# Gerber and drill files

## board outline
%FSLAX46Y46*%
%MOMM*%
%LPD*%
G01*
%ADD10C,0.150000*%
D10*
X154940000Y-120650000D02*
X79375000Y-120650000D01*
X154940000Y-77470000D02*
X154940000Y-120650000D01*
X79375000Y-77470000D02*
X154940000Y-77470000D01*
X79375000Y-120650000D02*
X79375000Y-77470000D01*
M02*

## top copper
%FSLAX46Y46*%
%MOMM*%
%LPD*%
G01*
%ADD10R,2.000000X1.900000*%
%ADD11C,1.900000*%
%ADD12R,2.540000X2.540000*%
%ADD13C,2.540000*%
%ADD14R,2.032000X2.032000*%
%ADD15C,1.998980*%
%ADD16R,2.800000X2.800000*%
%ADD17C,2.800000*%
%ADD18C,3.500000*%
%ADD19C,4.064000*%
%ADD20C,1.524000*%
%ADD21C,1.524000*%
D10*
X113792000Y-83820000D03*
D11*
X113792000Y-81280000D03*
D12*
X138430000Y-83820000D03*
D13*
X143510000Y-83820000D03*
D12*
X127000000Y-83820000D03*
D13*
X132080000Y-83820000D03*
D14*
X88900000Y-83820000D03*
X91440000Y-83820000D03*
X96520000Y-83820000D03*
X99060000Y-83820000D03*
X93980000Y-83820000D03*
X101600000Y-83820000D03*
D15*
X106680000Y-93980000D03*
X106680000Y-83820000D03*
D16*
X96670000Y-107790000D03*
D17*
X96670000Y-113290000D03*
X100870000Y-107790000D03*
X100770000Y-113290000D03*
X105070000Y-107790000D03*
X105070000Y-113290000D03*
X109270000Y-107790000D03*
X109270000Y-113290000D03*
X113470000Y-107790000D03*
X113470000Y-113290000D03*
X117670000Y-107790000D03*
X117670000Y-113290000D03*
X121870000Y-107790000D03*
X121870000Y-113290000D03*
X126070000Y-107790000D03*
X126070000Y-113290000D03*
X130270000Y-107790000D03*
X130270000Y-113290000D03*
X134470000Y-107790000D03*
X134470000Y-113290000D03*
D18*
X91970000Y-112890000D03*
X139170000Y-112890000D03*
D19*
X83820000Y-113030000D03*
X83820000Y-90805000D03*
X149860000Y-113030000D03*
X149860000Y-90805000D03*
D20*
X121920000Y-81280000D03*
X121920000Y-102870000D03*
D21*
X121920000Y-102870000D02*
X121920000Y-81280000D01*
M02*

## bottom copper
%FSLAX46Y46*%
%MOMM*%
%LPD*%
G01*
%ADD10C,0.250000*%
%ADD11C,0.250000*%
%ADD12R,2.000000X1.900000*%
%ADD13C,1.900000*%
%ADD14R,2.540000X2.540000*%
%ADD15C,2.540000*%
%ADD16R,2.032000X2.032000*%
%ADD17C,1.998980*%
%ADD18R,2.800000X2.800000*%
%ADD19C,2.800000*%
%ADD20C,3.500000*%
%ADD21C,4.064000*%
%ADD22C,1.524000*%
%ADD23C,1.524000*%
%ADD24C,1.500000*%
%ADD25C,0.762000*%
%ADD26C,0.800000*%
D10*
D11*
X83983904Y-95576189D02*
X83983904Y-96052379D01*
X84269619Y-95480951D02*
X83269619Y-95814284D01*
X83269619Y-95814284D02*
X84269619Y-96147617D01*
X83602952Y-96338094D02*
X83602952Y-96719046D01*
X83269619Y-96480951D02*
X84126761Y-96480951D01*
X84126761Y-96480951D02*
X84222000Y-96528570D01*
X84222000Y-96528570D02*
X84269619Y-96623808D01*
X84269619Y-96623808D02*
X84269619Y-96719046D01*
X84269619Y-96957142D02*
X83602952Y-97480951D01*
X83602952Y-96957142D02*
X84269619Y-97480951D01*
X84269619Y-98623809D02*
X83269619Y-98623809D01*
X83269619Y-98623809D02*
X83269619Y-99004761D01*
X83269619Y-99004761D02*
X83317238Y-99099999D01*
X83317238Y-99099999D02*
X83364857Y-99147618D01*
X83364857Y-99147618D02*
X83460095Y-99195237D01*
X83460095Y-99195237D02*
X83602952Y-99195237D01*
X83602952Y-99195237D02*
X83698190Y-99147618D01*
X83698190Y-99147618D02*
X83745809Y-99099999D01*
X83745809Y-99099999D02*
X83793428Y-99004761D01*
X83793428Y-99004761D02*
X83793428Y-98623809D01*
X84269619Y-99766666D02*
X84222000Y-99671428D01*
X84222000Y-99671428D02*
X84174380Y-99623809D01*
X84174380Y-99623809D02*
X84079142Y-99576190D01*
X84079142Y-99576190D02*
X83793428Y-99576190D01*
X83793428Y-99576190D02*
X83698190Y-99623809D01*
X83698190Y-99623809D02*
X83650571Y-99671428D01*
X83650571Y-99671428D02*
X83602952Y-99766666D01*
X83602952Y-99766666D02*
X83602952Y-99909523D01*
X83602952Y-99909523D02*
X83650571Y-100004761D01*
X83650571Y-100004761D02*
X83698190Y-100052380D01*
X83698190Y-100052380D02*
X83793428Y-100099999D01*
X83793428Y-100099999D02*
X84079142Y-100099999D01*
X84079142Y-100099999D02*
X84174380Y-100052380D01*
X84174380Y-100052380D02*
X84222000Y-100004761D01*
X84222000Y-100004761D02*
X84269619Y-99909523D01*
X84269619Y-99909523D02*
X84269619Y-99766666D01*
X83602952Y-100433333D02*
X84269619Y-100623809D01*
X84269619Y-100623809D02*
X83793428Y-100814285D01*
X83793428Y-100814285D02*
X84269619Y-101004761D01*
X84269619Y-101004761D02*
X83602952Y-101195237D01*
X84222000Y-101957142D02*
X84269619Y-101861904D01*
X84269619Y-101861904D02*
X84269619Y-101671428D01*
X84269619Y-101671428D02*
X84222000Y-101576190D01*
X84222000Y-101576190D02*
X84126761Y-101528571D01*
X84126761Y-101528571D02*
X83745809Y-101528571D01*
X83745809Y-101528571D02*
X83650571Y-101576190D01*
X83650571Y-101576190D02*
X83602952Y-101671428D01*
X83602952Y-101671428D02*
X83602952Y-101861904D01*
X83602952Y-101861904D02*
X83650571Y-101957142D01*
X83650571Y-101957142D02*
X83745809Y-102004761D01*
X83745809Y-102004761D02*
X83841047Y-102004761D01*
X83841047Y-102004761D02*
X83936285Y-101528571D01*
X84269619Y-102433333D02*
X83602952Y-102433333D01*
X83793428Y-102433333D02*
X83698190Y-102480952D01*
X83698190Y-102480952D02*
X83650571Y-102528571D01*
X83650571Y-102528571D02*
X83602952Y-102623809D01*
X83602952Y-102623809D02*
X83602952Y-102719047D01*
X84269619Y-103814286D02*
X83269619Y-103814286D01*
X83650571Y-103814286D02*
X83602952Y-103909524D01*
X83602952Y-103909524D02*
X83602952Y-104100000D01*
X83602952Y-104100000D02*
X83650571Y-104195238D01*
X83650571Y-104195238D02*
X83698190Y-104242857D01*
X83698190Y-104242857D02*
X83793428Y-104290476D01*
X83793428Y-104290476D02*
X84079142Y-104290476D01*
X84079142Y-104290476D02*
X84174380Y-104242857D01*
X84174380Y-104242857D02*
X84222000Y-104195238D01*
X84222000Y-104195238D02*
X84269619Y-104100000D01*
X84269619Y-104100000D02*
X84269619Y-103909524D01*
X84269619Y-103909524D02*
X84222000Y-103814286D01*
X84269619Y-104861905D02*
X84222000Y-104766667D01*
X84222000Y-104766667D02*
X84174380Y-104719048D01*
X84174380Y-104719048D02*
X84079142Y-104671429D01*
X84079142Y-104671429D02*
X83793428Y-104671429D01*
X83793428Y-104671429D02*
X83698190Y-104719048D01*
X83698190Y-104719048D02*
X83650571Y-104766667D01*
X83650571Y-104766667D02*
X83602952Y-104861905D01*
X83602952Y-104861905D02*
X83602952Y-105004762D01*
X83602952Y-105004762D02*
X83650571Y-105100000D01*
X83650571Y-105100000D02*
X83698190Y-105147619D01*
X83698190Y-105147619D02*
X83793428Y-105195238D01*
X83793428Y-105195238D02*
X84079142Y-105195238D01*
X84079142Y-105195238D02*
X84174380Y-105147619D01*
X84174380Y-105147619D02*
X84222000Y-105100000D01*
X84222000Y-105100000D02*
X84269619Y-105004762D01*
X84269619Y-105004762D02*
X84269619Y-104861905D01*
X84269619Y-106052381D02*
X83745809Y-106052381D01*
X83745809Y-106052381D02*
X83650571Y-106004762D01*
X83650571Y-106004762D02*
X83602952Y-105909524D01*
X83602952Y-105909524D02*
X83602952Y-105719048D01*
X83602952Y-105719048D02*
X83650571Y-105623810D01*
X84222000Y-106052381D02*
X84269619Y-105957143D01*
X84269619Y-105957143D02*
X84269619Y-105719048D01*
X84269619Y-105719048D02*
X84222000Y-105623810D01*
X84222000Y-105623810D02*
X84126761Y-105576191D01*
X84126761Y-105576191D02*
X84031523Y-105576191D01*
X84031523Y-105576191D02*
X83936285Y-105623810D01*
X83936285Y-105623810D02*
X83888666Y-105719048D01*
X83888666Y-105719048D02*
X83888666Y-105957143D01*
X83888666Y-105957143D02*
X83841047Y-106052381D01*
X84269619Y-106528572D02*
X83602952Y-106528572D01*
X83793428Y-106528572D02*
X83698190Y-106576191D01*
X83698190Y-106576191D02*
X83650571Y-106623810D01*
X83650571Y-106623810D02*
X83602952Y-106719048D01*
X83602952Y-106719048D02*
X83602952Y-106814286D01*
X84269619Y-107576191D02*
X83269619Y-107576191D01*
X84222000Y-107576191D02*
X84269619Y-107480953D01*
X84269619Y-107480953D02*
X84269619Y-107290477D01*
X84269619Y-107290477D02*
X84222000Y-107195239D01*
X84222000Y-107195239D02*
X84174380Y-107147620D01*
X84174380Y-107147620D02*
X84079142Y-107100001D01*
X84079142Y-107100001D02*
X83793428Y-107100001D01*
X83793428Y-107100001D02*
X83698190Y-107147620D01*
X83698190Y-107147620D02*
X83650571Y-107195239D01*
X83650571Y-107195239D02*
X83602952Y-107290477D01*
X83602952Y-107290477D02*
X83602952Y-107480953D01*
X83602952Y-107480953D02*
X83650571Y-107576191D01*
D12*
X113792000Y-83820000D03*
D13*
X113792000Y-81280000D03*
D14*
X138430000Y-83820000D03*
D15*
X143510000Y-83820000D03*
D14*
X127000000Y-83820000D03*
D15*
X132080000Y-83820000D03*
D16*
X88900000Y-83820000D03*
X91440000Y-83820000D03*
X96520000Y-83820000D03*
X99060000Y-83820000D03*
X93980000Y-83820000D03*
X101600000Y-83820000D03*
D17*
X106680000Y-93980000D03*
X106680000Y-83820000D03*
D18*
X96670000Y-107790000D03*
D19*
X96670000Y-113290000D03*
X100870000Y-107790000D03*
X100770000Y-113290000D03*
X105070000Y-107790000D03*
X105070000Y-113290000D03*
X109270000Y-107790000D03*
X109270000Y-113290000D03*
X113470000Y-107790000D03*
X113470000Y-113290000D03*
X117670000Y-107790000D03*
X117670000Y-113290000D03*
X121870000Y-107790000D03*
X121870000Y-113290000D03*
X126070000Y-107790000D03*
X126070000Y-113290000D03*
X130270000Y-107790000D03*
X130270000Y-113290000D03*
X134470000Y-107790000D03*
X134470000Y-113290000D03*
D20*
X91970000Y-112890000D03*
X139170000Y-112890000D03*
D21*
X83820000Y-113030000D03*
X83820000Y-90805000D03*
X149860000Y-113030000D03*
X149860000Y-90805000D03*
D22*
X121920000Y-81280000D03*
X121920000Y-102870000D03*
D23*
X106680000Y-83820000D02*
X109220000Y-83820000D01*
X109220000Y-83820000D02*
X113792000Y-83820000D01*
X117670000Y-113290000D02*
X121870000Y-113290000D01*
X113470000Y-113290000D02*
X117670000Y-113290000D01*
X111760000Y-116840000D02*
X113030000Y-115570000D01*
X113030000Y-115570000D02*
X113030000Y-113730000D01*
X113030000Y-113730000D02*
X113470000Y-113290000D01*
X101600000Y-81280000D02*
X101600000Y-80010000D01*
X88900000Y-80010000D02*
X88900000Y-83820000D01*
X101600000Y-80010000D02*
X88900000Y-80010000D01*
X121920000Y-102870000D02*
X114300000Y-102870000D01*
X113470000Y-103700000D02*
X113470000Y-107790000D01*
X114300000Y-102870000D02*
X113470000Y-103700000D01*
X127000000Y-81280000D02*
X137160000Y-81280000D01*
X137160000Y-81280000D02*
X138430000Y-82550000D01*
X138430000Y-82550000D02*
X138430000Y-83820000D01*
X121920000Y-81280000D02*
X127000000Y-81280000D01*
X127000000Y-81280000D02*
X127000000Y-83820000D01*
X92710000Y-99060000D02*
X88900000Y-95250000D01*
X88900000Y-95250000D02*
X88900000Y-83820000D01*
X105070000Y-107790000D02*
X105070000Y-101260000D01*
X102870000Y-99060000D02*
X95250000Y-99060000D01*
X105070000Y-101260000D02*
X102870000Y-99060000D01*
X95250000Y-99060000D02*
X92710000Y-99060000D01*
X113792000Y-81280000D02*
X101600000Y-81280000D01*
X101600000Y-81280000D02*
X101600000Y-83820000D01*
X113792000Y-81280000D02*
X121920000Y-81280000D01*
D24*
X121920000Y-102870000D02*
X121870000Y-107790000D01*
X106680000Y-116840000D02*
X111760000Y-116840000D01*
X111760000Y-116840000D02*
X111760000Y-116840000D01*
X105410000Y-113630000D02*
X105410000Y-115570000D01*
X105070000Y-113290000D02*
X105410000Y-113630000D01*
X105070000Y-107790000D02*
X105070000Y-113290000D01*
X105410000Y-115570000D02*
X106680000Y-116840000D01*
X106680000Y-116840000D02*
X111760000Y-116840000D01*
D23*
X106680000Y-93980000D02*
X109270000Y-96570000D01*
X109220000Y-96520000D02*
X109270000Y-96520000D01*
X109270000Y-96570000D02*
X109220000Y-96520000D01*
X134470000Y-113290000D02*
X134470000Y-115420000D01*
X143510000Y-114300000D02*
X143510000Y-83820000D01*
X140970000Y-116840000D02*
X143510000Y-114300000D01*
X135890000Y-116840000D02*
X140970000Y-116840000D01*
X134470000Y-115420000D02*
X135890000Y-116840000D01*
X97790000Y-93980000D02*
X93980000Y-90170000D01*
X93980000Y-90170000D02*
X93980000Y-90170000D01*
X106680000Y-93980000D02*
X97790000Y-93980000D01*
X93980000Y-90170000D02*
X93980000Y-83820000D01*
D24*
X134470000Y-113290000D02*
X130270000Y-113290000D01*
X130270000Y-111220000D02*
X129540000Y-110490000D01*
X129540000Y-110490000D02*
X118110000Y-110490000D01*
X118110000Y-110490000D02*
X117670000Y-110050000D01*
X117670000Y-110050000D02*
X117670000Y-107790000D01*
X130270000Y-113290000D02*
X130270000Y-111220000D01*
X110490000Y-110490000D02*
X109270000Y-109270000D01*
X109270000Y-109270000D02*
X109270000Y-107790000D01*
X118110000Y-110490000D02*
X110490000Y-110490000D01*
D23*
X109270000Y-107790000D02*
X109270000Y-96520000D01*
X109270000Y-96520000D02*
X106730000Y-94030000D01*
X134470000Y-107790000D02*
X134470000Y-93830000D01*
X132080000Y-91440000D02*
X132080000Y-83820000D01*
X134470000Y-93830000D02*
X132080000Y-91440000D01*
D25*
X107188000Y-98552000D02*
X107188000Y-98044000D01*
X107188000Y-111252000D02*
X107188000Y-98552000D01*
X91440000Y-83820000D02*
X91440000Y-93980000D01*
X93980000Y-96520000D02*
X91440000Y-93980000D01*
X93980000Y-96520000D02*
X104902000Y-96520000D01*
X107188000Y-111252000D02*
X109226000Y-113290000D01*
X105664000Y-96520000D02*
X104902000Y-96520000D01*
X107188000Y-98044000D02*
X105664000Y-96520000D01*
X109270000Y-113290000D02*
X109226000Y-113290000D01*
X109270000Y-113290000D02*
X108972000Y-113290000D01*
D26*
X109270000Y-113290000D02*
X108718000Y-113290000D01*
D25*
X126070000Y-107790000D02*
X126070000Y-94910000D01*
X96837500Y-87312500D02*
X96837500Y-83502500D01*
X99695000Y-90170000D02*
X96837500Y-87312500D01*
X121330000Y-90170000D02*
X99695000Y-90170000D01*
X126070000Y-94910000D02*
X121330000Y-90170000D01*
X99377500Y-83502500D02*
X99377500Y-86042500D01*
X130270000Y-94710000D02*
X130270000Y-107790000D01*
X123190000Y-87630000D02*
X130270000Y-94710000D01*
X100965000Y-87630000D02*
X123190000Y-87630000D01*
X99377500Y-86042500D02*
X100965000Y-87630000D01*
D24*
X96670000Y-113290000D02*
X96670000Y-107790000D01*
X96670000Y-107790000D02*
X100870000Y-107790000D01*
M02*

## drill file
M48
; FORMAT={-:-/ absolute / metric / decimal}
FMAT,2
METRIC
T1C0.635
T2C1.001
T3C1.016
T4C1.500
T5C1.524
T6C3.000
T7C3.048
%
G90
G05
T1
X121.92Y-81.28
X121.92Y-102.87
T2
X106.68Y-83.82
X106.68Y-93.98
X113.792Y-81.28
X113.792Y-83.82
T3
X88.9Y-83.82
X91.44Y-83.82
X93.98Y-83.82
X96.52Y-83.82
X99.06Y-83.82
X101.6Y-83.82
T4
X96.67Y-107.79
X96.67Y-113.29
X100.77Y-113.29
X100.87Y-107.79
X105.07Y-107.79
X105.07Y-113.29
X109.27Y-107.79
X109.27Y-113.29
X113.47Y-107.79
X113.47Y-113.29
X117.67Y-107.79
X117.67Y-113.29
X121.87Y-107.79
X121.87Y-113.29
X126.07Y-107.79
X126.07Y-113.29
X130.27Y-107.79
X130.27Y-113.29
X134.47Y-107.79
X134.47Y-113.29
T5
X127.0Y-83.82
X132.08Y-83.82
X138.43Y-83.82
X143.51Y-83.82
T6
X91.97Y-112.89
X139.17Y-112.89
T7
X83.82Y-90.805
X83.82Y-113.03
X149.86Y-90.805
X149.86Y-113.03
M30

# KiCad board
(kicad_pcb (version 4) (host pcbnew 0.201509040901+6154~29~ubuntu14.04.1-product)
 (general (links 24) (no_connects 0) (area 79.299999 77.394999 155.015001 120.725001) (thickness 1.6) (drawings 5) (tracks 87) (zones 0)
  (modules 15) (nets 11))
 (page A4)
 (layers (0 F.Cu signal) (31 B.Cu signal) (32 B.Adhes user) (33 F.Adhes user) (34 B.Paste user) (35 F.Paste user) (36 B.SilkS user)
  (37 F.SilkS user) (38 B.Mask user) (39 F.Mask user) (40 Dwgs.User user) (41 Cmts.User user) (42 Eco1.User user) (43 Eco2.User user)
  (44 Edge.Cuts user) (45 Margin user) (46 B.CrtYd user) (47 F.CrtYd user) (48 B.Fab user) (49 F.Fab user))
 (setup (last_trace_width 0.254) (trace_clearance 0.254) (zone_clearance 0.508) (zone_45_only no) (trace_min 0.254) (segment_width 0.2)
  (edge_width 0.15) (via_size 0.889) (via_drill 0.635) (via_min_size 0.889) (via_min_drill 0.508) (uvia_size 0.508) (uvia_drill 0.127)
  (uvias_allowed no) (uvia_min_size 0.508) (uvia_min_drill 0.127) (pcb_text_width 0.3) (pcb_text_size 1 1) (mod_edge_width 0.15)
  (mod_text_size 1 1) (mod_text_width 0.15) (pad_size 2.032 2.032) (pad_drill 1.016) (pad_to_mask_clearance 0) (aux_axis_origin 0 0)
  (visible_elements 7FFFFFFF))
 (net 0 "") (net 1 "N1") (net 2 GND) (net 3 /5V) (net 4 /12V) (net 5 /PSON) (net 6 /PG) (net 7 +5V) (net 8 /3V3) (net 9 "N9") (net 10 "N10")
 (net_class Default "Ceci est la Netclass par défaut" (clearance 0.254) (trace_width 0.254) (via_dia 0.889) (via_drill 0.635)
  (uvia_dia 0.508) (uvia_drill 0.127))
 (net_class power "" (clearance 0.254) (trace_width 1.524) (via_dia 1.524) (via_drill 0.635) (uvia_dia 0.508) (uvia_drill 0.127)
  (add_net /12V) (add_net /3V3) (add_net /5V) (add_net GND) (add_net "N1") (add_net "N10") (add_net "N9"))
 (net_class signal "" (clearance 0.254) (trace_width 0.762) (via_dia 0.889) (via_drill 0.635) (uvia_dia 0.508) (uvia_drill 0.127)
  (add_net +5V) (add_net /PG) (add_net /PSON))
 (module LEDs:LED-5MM (layer F.Cu) (at 113.792 83.82 90)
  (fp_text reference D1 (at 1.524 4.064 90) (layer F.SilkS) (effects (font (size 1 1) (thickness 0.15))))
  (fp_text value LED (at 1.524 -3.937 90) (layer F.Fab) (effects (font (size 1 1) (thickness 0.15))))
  (pad 1 thru_hole rect (at 0 0 180) (size 2 1.9) (drill 1.00076) (layers *.Cu *.Mask F.SilkS) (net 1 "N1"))
  (pad 2 thru_hole circle (at 2.54 0 90) (size 1.9 1.9) (drill 1.00076) (layers *.Cu *.Mask F.SilkS) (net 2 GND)))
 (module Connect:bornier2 (layer F.Cu) (at 140.97 83.82)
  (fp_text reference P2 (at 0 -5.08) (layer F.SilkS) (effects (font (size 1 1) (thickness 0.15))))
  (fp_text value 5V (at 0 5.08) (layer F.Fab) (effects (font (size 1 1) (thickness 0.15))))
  (pad 1 thru_hole rect (at -2.54 0) (size 2.54 2.54) (drill 1.524) (layers *.Cu *.Mask F.SilkS) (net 2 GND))
  (pad 2 thru_hole circle (at 2.54 0) (size 2.54 2.54) (drill 1.524) (layers *.Cu *.Mask F.SilkS) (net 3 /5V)))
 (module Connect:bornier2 (layer F.Cu) (at 129.54 83.82)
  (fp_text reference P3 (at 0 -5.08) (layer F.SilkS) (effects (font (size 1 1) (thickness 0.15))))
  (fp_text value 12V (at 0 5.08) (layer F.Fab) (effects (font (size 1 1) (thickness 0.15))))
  (pad 1 thru_hole rect (at -2.54 0) (size 2.54 2.54) (drill 1.524) (layers *.Cu *.Mask F.SilkS) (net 2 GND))
  (pad 2 thru_hole circle (at 2.54 0) (size 2.54 2.54) (drill 1.524) (layers *.Cu *.Mask F.SilkS) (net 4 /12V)))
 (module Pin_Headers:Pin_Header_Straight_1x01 (layer F.Cu) (at 88.9 83.82)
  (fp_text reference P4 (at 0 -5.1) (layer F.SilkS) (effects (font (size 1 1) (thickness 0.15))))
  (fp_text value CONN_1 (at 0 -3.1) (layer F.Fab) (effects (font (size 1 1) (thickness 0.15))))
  (pad 1 thru_hole rect (at 0 0) (size 2.032 2.032) (drill 1.016) (layers *.Cu *.Mask F.SilkS) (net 2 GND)))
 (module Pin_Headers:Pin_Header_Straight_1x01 (layer F.Cu) (at 91.44 83.82)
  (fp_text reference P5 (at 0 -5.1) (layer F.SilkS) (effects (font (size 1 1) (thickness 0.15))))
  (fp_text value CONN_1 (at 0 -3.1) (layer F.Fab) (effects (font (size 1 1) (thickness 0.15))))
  (pad 1 thru_hole rect (at 0 0) (size 2.032 2.032) (drill 1.016) (layers *.Cu *.Mask F.SilkS) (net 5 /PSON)))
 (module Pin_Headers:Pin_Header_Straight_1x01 (layer F.Cu) (at 96.52 83.82)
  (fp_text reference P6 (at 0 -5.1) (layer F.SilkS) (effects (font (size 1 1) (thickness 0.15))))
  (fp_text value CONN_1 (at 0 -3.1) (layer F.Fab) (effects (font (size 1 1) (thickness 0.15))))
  (pad 1 thru_hole rect (at 0 0) (size 2.032 2.032) (drill 1.016) (layers *.Cu *.Mask F.SilkS) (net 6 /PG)))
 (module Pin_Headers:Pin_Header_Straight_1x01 (layer F.Cu) (at 99.06 83.82)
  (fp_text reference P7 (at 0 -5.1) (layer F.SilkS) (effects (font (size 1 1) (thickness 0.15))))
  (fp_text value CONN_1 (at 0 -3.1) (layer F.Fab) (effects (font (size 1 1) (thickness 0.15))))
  (pad 1 thru_hole rect (at 0 0) (size 2.032 2.032) (drill 1.016) (layers *.Cu *.Mask F.SilkS) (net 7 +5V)))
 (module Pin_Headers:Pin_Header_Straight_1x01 (layer F.Cu) (at 93.98 83.82)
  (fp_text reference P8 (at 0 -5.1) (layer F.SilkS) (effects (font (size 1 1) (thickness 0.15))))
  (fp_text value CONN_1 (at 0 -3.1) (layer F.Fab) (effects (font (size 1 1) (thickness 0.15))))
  (pad 1 thru_hole rect (at 0 0) (size 2.032 2.032) (drill 1.016) (layers *.Cu *.Mask F.SilkS) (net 3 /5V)))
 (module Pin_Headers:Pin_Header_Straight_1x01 (layer F.Cu) (at 101.6 83.82)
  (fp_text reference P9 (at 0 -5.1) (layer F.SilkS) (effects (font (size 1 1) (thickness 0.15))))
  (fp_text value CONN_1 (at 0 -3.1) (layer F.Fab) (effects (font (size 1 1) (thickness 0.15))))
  (pad 1 thru_hole rect (at 0 0) (size 2.032 2.032) (drill 1.016) (layers *.Cu *.Mask F.SilkS) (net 2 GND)))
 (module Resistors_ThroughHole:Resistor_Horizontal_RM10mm (layer F.Cu) (at 106.68 88.9 90)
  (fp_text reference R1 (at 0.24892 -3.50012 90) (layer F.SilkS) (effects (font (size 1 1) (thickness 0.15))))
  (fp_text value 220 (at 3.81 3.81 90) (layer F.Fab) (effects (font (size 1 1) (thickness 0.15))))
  (pad 1 thru_hole circle (at -5.08 0 90) (size 1.99898 1.99898) (drill 1.00076) (layers *.Cu *.SilkS *.Mask) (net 3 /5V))
  (pad 2 thru_hole circle (at 5.08 0 90) (size 1.99898 1.99898) (drill 1.00076) (layers *.Cu *.SilkS *.Mask) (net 1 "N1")))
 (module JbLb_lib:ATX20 (layer F.Cu) (at 115.57 110.49 180)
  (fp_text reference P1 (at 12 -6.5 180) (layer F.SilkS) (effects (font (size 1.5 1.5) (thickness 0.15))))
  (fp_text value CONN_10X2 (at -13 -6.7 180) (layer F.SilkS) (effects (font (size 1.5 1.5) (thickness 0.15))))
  (pad 1 thru_hole rect (at 18.9 2.7 180) (size 2.8 2.8) (drill 1.5) (layers *.Cu *.Mask F.SilkS) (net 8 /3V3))
  (pad 2 thru_hole circle (at 18.9 -2.8 180) (size 2.8 2.8) (drill 1.5) (layers *.Cu *.Mask F.SilkS) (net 8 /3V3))
  (pad 3 thru_hole circle (at 14.7 2.7 180) (size 2.8 2.8) (drill 1.5) (layers *.Cu *.Mask F.SilkS) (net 8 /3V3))
  (pad 4 thru_hole circle (at 14.8 -2.8 180) (size 2.8 2.8) (drill 1.5) (layers *.Cu *.Mask F.SilkS) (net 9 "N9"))
  (pad 5 thru_hole circle (at 10.5 2.7 180) (size 2.8 2.8) (drill 1.5) (layers *.Cu *.Mask F.SilkS) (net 2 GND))
  (pad 6 thru_hole circle (at 10.5 -2.8 180) (size 2.8 2.8) (drill 1.5) (layers *.Cu *.Mask F.SilkS) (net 2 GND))
  (pad 7 thru_hole circle (at 6.3 2.7 180) (size 2.8 2.8) (drill 1.5) (layers *.Cu *.Mask F.SilkS) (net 3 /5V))
  (pad 8 thru_hole circle (at 6.3 -2.8 180) (size 2.8 2.8) (drill 1.5) (layers *.Cu *.Mask F.SilkS) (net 5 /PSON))
  (pad 9 thru_hole circle (at 2.1 2.7 180) (size 2.8 2.8) (drill 1.5) (layers *.Cu *.Mask F.SilkS) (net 2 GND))
  (pad 10 thru_hole circle (at 2.1 -2.8 180) (size 2.8 2.8) (drill 1.5) (layers *.Cu *.Mask F.SilkS) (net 2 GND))
  (pad 11 thru_hole circle (at -2.1 2.7 180) (size 2.8 2.8) (drill 1.5) (layers *.Cu *.Mask F.SilkS) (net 3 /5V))
  (pad 12 thru_hole circle (at -2.1 -2.8 180) (size 2.8 2.8) (drill 1.5) (layers *.Cu *.Mask F.SilkS) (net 2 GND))
  (pad 13 thru_hole circle (at -6.3 2.7 180) (size 2.8 2.8) (drill 1.5) (layers *.Cu *.Mask F.SilkS) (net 2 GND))
  (pad 14 thru_hole circle (at -6.3 -2.8 180) (size 2.8 2.8) (drill 1.5) (layers *.Cu *.Mask F.SilkS) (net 2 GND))
  (pad 15 thru_hole circle (at -10.5 2.7 180) (size 2.8 2.8) (drill 1.5) (layers *.Cu *.Mask F.SilkS) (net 6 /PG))
  (pad 16 thru_hole circle (at -10.5 -2.8 180) (size 2.8 2.8) (drill 1.5) (layers *.Cu *.Mask F.SilkS) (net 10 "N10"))
  (pad 17 thru_hole circle (at -14.7 2.7 180) (size 2.8 2.8) (drill 1.5) (layers *.Cu *.Mask F.SilkS) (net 7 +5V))
  (pad 18 thru_hole circle (at -14.7 -2.8 180) (size 2.8 2.8) (drill 1.5) (layers *.Cu *.Mask F.SilkS) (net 3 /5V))
  (pad 19 thru_hole circle (at -18.9 2.7 180) (size 2.8 2.8) (drill 1.5) (layers *.Cu *.Mask F.SilkS) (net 4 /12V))
  (pad 20 thru_hole circle (at -18.9 -2.8 180) (size 2.8 2.8) (drill 1.5) (layers *.Cu *.Mask F.SilkS) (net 3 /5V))
  (pad 21 thru_hole circle (at 23.6 -2.4 180) (size 3.5 3.5) (drill 3) (layers *.Cu *.Mask F.SilkS))
  (pad 22 thru_hole circle (at -23.6 -2.4 180) (size 3.5 3.5) (drill 3) (layers *.Cu *.Mask F.SilkS)))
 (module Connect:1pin (layer F.Cu) (at 83.82 113.03 90)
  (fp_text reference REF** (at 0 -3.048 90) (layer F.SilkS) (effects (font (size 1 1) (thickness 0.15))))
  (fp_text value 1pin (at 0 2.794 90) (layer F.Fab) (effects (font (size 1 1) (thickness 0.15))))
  (pad 1 thru_hole circle (at 0 0 90) (size 4.064 4.064) (drill 3.048) (layers *.Cu *.Mask F.SilkS)))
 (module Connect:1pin (layer F.Cu) (at 83.82 90.805 90)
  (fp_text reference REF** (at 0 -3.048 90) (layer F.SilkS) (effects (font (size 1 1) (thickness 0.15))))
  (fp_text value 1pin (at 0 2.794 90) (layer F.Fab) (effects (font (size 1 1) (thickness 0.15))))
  (pad 1 thru_hole circle (at 0 0 90) (size 4.064 4.064) (drill 3.048) (layers *.Cu *.Mask F.SilkS)))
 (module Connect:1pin (layer F.Cu) (at 149.86 113.03 90)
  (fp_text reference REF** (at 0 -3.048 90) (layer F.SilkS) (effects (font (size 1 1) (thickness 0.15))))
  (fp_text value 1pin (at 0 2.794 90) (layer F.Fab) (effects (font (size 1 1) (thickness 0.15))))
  (pad 1 thru_hole circle (at 0 0 90) (size 4.064 4.064) (drill 3.048) (layers *.Cu *.Mask F.SilkS)))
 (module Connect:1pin (layer F.Cu) (at 149.86 90.805 90)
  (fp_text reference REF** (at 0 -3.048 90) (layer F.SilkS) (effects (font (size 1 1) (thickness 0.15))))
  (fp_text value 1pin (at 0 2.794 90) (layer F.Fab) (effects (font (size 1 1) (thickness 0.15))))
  (pad 1 thru_hole circle (at 0 0 90) (size 4.064 4.064) (drill 3.048) (layers *.Cu *.Mask F.SilkS)))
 (gr_line (start 154.94 120.65) (end 79.375 120.65) (angle 90) (layer Edge.Cuts) (width 0.15))
 (gr_line (start 154.94 77.47) (end 154.94 120.65) (angle 90) (layer Edge.Cuts) (width 0.15))
 (gr_line (start 79.375 77.47) (end 154.94 77.47) (angle 90) (layer Edge.Cuts) (width 0.15))
 (gr_line (start 79.375 120.65) (end 79.375 77.47) (angle 90) (layer Edge.Cuts) (width 0.15))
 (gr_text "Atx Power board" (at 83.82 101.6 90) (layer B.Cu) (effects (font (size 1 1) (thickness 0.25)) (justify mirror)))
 (segment (start 106.68 83.82) (end 109.22 83.82) (width 1.524) (layer B.Cu) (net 1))
 (segment (start 109.22 83.82) (end 113.792 83.82) (width 1.524) (layer B.Cu) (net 1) (status 30))
 (segment (start 117.67 113.29) (end 121.87 113.29) (width 1.524) (layer B.Cu) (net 2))
 (segment (start 113.47 113.29) (end 117.67 113.29) (width 1.524) (layer B.Cu) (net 2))
 (segment (start 111.76 116.84) (end 113.03 115.57) (width 1.524) (layer B.Cu) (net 2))
 (segment (start 113.03 115.57) (end 113.03 113.73) (width 1.524) (layer B.Cu) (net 2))
 (segment (start 113.03 113.73) (end 113.47 113.29) (width 1.524) (layer B.Cu) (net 2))
 (segment (start 101.6 81.28) (end 101.6 80.01) (width 1.524) (layer B.Cu) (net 2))
 (segment (start 88.9 80.01) (end 88.9 83.82) (width 1.524) (layer B.Cu) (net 2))
 (segment (start 101.6 80.01) (end 88.9 80.01) (width 1.524) (layer B.Cu) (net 2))
 (segment (start 121.92 102.87) (end 114.3 102.87) (width 1.524) (layer B.Cu) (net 2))
 (segment (start 113.47 103.7) (end 113.47 107.79) (width 1.524) (layer B.Cu) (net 2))
 (segment (start 114.3 102.87) (end 113.47 103.7) (width 1.524) (layer B.Cu) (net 2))
 (segment (start 127 81.28) (end 137.16 81.28) (width 1.524) (layer B.Cu) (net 2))
 (segment (start 137.16 81.28) (end 138.43 82.55) (width 1.524) (layer B.Cu) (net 2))
 (segment (start 138.43 82.55) (end 138.43 83.82) (width 1.524) (layer B.Cu) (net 2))
 (segment (start 121.92 81.28) (end 127 81.28) (width 1.524) (layer B.Cu) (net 2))
 (segment (start 127 81.28) (end 127 83.82) (width 1.524) (layer B.Cu) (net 2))
 (segment (start 92.71 99.06) (end 88.9 95.25) (width 1.524) (layer B.Cu) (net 2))
 (segment (start 88.9 95.25) (end 88.9 83.82) (width 1.524) (layer B.Cu) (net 2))
 (segment (start 105.07 107.79) (end 105.07 101.26) (width 1.524) (layer B.Cu) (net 2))
 (segment (start 102.87 99.06) (end 95.25 99.06) (width 1.524) (layer B.Cu) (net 2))
 (segment (start 105.07 101.26) (end 102.87 99.06) (width 1.524) (layer B.Cu) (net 2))
 (segment (start 95.25 99.06) (end 92.71 99.06) (width 1.524) (layer B.Cu) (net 2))
 (segment (start 113.792 81.28) (end 101.6 81.28) (width 1.524) (layer B.Cu) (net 2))
 (segment (start 101.6 81.28) (end 101.6 83.82) (width 1.524) (layer B.Cu) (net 2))
 (segment (start 113.792 81.28) (end 121.92 81.28) (width 1.524) (layer B.Cu) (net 2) (status 10))
 (segment (start 121.92 102.87) (end 121.87 107.79) (width 1.5) (layer B.Cu) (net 2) (status 20))
 (via (at 121.92 81.28) (size 1.524) (layers F.Cu B.Cu) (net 2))
 (segment (start 121.92 102.87) (end 121.92 81.28) (width 1.524) (layer F.Cu) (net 2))
 (via (at 121.92 102.87) (size 1.524) (layers F.Cu B.Cu) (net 2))
 (segment (start 106.68 116.84) (end 111.76 116.84) (width 1.5) (layer B.Cu) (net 2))
 (segment (start 111.76 116.84) (end 111.76 116.84) (width 1.5) (layer B.Cu) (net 2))
 (segment (start 105.41 113.63) (end 105.41 115.57) (width 1.5) (layer B.Cu) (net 2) (status 10))
 (segment (start 105.07 113.29) (end 105.41 113.63) (width 1.5) (layer B.Cu) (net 2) (status 30))
 (segment (start 105.07 107.79) (end 105.07 113.29) (width 1.5) (layer B.Cu) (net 2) (status 30))
 (segment (start 105.41 115.57) (end 106.68 116.84) (width 1.5) (layer B.Cu) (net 2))
 (segment (start 106.68 116.84) (end 111.76 116.84) (width 1.5) (layer B.Cu) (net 2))
 (segment (start 106.68 93.98) (end 109.27 96.57) (width 1.524) (layer B.Cu) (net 3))
 (segment (start 109.22 96.52) (end 109.27 96.52) (width 1.524) (layer B.Cu) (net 3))
 (segment (start 109.27 96.57) (end 109.22 96.52) (width 1.524) (layer B.Cu) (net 3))
 (segment (start 134.47 113.29) (end 134.47 115.42) (width 1.524) (layer B.Cu) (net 3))
 (segment (start 143.51 114.3) (end 143.51 83.82) (width 1.524) (layer B.Cu) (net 3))
 (segment (start 140.97 116.84) (end 143.51 114.3) (width 1.524) (layer B.Cu) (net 3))
 (segment (start 135.89 116.84) (end 140.97 116.84) (width 1.524) (layer B.Cu) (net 3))
 (segment (start 134.47 115.42) (end 135.89 116.84) (width 1.524) (layer B.Cu) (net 3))
 (segment (start 97.79 93.98) (end 93.98 90.17) (width 1.524) (layer B.Cu) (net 3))
 (segment (start 93.98 90.17) (end 93.98 90.17) (width 1.524) (layer B.Cu) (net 3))
 (segment (start 106.68 93.98) (end 97.79 93.98) (width 1.524) (layer B.Cu) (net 3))
 (segment (start 93.98 90.17) (end 93.98 83.82) (width 1.524) (layer B.Cu) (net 3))
 (segment (start 134.47 113.29) (end 130.27 113.29) (width 1.5) (layer B.Cu) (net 3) (status 30))
 (segment (start 130.27 111.22) (end 129.54 110.49) (width 1.5) (layer B.Cu) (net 3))
 (segment (start 129.54 110.49) (end 118.11 110.49) (width 1.5) (layer B.Cu) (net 3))
 (segment (start 118.11 110.49) (end 117.67 110.05) (width 1.5) (layer B.Cu) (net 3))
 (segment (start 117.67 110.05) (end 117.67 107.79) (width 1.5) (layer B.Cu) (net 3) (status 20))
 (segment (start 130.27 113.29) (end 130.27 111.22) (width 1.5) (layer B.Cu) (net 3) (status 10))
 (segment (start 110.49 110.49) (end 109.27 109.27) (width 1.5) (layer B.Cu) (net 3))
 (segment (start 109.27 109.27) (end 109.27 107.79) (width 1.5) (layer B.Cu) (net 3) (status 20))
 (segment (start 118.11 110.49) (end 110.49 110.49) (width 1.5) (layer B.Cu) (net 3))
 (segment (start 109.27 107.79) (end 109.27 96.52) (width 1.524) (layer B.Cu) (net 3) (status 30))
 (segment (start 109.27 96.52) (end 106.73 94.03) (width 1.524) (layer B.Cu) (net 3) (status 30))
 (segment (start 134.47 107.79) (end 134.47 93.83) (width 1.524) (layer B.Cu) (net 4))
 (segment (start 132.08 91.44) (end 132.08 83.82) (width 1.524) (layer B.Cu) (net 4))
 (segment (start 134.47 93.83) (end 132.08 91.44) (width 1.524) (layer B.Cu) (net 4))
 (segment (start 107.188 98.552) (end 107.188 98.044) (width 0.762) (layer B.Cu) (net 5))
 (segment (start 107.188 111.252) (end 107.188 98.552) (width 0.762) (layer B.Cu) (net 5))
 (segment (start 91.44 83.82) (end 91.44 93.98) (width 0.762) (layer B.Cu) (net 5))
 (segment (start 93.98 96.52) (end 91.44 93.98) (width 0.762) (layer B.Cu) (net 5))
 (segment (start 93.98 96.52) (end 104.902 96.52) (width 0.762) (layer B.Cu) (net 5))
 (segment (start 107.188 111.252) (end 109.226 113.29) (width 0.762) (layer B.Cu) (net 5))
 (segment (start 105.664 96.52) (end 104.902 96.52) (width 0.762) (layer B.Cu) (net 5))
 (segment (start 107.188 98.044) (end 105.664 96.52) (width 0.762) (layer B.Cu) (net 5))
 (segment (start 109.27 113.29) (end 109.226 113.29) (width 0.762) (layer B.Cu) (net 5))
 (segment (start 109.27 113.29) (end 108.972 113.29) (width 0.762) (layer B.Cu) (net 5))
 (segment (start 109.27 113.29) (end 108.718 113.29) (width 0.8) (layer B.Cu) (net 5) (status 30))
 (segment (start 126.07 107.79) (end 126.07 94.91) (width 0.762) (layer B.Cu) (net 6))
 (segment (start 96.8375 87.3125) (end 96.8375 83.5025) (width 0.762) (layer B.Cu) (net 6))
 (segment (start 99.695 90.17) (end 96.8375 87.3125) (width 0.762) (layer B.Cu) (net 6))
 (segment (start 121.33 90.17) (end 99.695 90.17) (width 0.762) (layer B.Cu) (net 6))
 (segment (start 126.07 94.91) (end 121.33 90.17) (width 0.762) (layer B.Cu) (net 6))
 (segment (start 99.3775 83.5025) (end 99.3775 86.0425) (width 0.762) (layer B.Cu) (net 7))
 (segment (start 130.27 94.71) (end 130.27 107.79) (width 0.762) (layer B.Cu) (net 7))
 (segment (start 123.19 87.63) (end 130.27 94.71) (width 0.762) (layer B.Cu) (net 7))
 (segment (start 100.965 87.63) (end 123.19 87.63) (width 0.762) (layer B.Cu) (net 7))
 (segment (start 99.3775 86.0425) (end 100.965 87.63) (width 0.762) (layer B.Cu) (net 7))
 (segment (start 96.67 113.29) (end 96.67 107.79) (width 1.5) (layer B.Cu) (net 8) (status 30))
 (segment (start 96.67 107.79) (end 100.87 107.79) (width 1.5) (layer B.Cu) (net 8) (status 30)))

